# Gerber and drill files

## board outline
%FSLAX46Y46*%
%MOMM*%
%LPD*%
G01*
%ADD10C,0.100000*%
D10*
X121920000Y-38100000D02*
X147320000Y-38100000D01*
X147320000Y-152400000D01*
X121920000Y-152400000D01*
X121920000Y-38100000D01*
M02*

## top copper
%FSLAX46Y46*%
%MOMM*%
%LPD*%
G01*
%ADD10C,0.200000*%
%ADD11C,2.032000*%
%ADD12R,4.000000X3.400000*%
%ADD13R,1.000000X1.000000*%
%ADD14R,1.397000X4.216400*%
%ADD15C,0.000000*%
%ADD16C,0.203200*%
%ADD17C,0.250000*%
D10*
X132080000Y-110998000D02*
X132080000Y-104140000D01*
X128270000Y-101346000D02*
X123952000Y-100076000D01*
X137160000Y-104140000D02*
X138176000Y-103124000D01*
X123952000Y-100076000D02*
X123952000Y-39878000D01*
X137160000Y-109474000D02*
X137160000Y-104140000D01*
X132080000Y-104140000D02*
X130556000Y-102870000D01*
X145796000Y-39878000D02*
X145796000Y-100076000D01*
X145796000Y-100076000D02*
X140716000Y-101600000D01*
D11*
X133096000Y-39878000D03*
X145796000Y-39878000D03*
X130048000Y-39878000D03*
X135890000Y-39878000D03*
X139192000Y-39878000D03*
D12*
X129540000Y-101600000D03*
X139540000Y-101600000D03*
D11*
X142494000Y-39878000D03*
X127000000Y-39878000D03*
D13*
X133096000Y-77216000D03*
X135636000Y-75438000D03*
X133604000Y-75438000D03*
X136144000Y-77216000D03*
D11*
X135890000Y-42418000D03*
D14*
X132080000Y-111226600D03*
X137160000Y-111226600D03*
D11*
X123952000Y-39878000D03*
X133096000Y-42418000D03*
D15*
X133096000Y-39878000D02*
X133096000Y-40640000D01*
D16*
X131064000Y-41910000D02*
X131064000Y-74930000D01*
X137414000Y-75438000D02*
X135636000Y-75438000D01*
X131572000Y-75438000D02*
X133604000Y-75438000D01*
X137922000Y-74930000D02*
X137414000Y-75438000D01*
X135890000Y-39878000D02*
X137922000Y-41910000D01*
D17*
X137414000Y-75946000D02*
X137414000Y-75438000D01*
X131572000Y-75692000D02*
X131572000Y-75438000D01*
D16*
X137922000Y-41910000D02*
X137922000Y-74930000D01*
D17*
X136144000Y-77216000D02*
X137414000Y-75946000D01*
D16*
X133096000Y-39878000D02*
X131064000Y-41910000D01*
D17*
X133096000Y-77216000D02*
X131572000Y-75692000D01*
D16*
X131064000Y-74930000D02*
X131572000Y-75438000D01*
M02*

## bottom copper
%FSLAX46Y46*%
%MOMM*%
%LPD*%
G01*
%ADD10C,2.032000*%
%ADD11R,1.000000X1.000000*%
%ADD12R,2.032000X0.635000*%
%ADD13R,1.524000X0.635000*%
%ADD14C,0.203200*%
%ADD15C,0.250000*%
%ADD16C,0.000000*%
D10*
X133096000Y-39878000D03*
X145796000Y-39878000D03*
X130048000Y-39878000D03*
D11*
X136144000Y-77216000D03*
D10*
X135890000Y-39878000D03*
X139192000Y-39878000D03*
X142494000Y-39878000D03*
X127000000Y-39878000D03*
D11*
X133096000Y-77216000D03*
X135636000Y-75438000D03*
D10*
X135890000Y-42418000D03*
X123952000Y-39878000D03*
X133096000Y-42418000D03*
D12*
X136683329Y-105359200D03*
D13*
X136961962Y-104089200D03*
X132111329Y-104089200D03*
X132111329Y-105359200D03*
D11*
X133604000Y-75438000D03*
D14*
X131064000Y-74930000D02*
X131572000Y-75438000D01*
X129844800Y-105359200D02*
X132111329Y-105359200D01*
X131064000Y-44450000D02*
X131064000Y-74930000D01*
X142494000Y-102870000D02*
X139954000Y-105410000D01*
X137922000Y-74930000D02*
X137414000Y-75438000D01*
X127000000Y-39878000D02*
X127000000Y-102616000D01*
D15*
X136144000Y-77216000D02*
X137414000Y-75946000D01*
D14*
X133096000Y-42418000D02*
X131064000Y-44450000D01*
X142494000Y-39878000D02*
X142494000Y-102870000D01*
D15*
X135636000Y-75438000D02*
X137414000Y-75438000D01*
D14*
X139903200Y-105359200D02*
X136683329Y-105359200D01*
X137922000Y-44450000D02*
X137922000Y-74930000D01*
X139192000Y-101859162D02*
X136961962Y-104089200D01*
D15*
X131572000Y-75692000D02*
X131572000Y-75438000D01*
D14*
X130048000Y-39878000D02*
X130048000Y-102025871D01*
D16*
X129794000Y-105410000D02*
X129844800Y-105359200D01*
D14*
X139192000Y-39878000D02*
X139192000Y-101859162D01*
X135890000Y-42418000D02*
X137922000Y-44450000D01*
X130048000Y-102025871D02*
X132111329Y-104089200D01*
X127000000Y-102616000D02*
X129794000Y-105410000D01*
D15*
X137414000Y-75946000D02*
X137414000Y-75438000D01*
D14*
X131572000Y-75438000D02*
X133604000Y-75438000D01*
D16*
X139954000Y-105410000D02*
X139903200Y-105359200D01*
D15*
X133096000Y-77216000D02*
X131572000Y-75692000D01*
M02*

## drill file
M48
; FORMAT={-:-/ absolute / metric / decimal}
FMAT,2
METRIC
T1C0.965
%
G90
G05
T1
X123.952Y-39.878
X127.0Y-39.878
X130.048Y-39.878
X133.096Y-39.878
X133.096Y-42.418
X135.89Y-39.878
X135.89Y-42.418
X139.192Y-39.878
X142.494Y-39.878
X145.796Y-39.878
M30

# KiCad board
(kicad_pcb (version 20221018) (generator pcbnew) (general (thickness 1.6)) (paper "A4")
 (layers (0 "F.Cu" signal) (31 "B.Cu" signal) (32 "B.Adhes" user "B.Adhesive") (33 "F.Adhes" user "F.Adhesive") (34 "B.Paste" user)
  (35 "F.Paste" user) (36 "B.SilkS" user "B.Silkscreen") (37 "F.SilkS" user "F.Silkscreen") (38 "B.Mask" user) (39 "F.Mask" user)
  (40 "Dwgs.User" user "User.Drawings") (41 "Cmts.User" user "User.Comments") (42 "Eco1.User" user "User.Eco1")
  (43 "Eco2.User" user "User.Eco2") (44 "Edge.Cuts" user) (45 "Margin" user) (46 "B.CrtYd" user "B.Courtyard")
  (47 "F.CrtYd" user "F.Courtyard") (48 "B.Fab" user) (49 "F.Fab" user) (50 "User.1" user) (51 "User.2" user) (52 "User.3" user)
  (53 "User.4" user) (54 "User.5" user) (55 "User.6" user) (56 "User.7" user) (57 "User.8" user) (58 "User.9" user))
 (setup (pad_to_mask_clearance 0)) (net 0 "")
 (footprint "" (layer "F.Cu") (at 133.096 52.578)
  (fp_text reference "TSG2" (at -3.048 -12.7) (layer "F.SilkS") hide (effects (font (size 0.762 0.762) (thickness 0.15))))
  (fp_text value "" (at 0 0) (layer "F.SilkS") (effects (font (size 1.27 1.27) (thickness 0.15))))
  (pad "1" thru_hole circle (at 0 -12.7) (size 2.032 2.032) (drill 0.9652) (layers "*.Cu" "*.Mask")))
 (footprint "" (layer "F.Cu") (at 145.796 39.878)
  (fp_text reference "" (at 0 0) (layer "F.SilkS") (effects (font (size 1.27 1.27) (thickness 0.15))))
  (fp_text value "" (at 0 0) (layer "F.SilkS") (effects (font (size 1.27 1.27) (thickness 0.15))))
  (pad "1" thru_hole circle (at 0 0) (size 2.032 2.032) (drill 0.9652) (layers "*.Cu" "*.Mask")))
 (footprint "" (layer "F.Cu") (at 130.048 39.878)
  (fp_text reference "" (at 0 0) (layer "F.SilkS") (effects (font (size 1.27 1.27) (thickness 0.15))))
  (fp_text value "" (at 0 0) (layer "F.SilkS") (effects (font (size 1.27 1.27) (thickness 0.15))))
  (pad "1" thru_hole circle (at 0 0) (size 2.032 2.032) (drill 0.9652) (layers "*.Cu" "*.Mask")))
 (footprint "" (layer "F.Cu") (at 136.144 77.216)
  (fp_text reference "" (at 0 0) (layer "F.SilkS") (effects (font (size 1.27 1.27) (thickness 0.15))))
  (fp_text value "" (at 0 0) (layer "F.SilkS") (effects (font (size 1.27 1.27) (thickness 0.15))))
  (pad "1" smd rect (at 0 0 180) (size 1 1) (layers "B.Cu" "B.Mask")))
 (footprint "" (layer "F.Cu") (at 135.89 52.578)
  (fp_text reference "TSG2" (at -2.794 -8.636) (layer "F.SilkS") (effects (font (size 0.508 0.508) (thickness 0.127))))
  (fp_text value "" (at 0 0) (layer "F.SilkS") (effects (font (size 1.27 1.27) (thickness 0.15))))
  (pad "1" thru_hole circle (at 0 -12.7) (size 2.032 2.032) (drill 0.9652) (layers "*.Cu" "*.Mask")))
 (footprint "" (layer "F.Cu") (at 139.192 39.878)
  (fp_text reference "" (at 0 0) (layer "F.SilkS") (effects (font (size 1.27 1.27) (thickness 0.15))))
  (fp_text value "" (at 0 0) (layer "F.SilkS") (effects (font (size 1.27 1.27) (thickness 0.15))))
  (pad "1" thru_hole circle (at 0 0) (size 2.032 2.032) (drill 0.9652) (layers "*.Cu" "*.Mask")))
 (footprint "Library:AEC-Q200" (layer "F.Cu") (at 134.62 107.95)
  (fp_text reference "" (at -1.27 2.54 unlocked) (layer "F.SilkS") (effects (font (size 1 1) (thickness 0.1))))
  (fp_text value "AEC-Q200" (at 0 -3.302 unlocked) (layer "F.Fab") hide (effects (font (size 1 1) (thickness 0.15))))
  (pad "1" smd rect (at -5.08 -6.35 180) (size 4 3.4) (layers "F.Cu" "F.Mask"))
  (pad "2" smd rect (at 4.92 -6.35 180) (size 4 3.4) (layers "F.Cu" "F.Mask")))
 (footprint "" (layer "F.Cu") (at 142.494 39.878)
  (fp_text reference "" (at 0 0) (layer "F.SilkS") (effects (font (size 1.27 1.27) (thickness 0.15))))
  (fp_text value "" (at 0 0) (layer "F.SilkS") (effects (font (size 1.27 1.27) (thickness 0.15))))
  (pad "1" thru_hole circle (at 0 0) (size 2.032 2.032) (drill 0.9652) (layers "*.Cu" "*.Mask")))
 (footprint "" (layer "F.Cu") (at 127 39.878)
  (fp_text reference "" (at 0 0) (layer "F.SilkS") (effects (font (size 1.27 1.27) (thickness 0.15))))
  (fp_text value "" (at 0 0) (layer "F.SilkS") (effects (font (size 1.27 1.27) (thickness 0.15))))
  (pad "1" thru_hole circle (at 0 0) (size 2.032 2.032) (drill 0.9652) (layers "*.Cu" "*.Mask")))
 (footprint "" (layer "F.Cu") (at 133.096 77.216)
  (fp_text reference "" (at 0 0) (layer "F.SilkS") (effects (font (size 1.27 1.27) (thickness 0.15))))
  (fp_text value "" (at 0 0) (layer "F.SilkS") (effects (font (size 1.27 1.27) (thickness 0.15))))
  (pad "1" smd rect (at 0 0) (size 1 1) (layers "F.Cu" "F.Mask")))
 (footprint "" (layer "F.Cu") (at 133.096 77.216)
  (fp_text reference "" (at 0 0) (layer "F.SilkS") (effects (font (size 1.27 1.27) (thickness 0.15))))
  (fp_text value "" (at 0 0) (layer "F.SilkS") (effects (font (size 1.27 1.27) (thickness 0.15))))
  (pad "1" smd rect (at 0 0 180) (size 1 1) (layers "B.Cu" "B.Mask")))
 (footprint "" (layer "F.Cu") (at 135.636 75.438)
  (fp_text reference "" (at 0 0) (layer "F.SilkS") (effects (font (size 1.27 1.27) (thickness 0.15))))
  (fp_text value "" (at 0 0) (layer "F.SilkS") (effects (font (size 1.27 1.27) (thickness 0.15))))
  (pad "1" smd rect (at 0 0) (size 1 1) (layers "F.Cu" "F.Mask")))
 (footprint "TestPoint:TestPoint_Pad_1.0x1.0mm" (layer "F.Cu") (at 133.604 75.438)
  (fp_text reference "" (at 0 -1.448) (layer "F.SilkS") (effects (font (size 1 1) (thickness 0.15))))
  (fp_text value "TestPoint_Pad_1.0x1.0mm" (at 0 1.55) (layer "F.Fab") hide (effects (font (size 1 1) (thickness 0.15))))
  (pad "1" smd rect (at 0 0) (size 1 1) (layers "F.Cu" "F.Mask")))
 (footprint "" (layer "F.Cu") (at 136.144 77.216)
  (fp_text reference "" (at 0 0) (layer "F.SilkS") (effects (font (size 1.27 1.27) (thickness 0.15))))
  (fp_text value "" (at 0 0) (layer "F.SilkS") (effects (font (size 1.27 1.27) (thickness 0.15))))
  (pad "1" smd rect (at 0 0) (size 1 1) (layers "F.Cu" "F.Mask")))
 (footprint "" (layer "F.Cu") (at 135.636 75.438)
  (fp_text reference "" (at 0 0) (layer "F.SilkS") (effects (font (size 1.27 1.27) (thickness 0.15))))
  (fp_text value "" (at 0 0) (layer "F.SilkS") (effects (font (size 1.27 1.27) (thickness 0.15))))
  (pad "1" smd rect (at 0 0 180) (size 1 1) (layers "B.Cu" "B.Mask")))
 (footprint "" (layer "F.Cu") (at 135.89 55.118)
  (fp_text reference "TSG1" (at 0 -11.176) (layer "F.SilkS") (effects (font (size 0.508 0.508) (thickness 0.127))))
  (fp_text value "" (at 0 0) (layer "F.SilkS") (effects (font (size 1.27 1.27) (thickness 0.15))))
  (pad "1" thru_hole circle (at 0 -12.7) (size 2.032 2.032) (drill 0.9652) (layers "*.Cu" "*.Mask")))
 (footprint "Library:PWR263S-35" (layer "F.Cu") (at 135.89 112.268)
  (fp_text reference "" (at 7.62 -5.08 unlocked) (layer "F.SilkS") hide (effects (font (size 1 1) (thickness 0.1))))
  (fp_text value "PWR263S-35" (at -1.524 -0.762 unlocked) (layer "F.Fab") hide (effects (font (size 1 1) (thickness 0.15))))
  (pad "1" smd rect (at -3.81 -1.0414) (size 1.397 4.2164) (layers "F.Cu" "F.Mask"))
  (pad "2" smd rect (at 1.27 -1.0414) (size 1.397 4.2164) (layers "F.Cu" "F.Mask")))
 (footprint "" (layer "F.Cu") (at 123.952 39.878)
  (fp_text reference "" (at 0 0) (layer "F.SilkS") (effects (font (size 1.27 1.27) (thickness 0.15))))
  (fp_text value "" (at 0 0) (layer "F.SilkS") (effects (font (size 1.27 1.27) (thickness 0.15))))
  (pad "1" thru_hole circle (at 0 0) (size 2.032 2.032) (drill 0.9652) (layers "*.Cu" "*.Mask")))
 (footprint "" (layer "F.Cu") (at 133.096 55.118)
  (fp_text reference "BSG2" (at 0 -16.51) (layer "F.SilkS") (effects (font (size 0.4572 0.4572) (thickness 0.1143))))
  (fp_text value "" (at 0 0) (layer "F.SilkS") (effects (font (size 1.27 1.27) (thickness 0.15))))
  (pad "1" thru_hole circle (at 0 -12.7) (size 2.032 2.032) (drill 0.9652) (layers "*.Cu" "*.Mask")))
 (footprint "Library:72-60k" (layer "B.Cu") (at 132.873329 109.1692 180)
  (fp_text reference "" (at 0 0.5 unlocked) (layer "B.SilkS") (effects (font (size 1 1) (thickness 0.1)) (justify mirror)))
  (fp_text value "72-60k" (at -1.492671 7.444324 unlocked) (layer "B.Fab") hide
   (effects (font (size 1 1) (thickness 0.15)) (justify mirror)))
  (pad "1" smd rect (at -3.81 3.81) (size 2.032 0.635) (layers "B.Cu" "B.Mask"))
  (pad "2" smd rect (at -4.088633 5.08) (size 1.524 0.635) (layers "B.Cu" "B.Mask"))
  (pad "3" smd rect (at 0.762 5.08) (size 1.524 0.635) (layers "B.Cu" "B.Mask"))
  (pad "4" smd rect (at 0.762 3.81) (size 1.524 0.635) (layers "B.Cu" "B.Mask")))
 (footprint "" (layer "B.Cu") (at 133.604 75.438 180)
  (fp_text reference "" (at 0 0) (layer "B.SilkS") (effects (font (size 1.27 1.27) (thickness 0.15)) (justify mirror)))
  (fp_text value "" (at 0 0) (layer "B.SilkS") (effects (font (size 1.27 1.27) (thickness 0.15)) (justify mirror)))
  (pad "1" smd rect (at 0 0 180) (size 1 1) (layers "B.Cu" "B.Mask")))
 (gr_line (start 132.08 110.998) (end 132.08 104.14) (stroke (width 0.2) (type default)) (layer "F.Cu"))
 (gr_line (start 128.27 101.346) (end 123.952 100.076) (stroke (width 0.2) (type default)) (layer "F.Cu"))
 (gr_line (start 137.16 104.14) (end 138.176 103.124) (stroke (width 0.2) (type default)) (layer "F.Cu"))
 (gr_line (start 123.952 100.076) (end 123.952 39.878) (stroke (width 0.2) (type default)) (layer "F.Cu"))
 (gr_line (start 137.16 109.474) (end 137.16 104.14) (stroke (width 0.2) (type default)) (layer "F.Cu"))
 (gr_line (start 132.08 104.14) (end 130.556 102.87) (stroke (width 0.2) (type default)) (layer "F.Cu"))
 (gr_line (start 145.796 39.878) (end 145.796 100.076) (stroke (width 0.2) (type default)) (layer "F.Cu"))
 (gr_line (start 145.796 100.076) (end 140.716 101.6) (stroke (width 0.2) (type default)) (layer "F.Cu"))
 (gr_rect (start 121.92 38.1) (end 147.32 152.4) (stroke (width 0.1) (type default)) (fill none) (layer "Edge.Cuts"))
 (segment (start 133.096 39.878) (end 133.096 40.64) (width 0) (layer "F.Cu") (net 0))
 (segment (start 131.064 41.91) (end 131.064 74.93) (width 0.2032) (layer "F.Cu") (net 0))
 (segment (start 137.414 75.438) (end 135.636 75.438) (width 0.2032) (layer "F.Cu") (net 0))
 (segment (start 131.572 75.438) (end 133.604 75.438) (width 0.2032) (layer "F.Cu") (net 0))
 (segment (start 137.922 74.93) (end 137.414 75.438) (width 0.2032) (layer "F.Cu") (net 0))
 (segment (start 135.89 39.878) (end 137.922 41.91) (width 0.2032) (layer "F.Cu") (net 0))
 (segment (start 137.414 75.946) (end 137.414 75.438) (width 0.25) (layer "F.Cu") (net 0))
 (segment (start 131.572 75.692) (end 131.572 75.438) (width 0.25) (layer "F.Cu") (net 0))
 (segment (start 137.922 41.91) (end 137.922 74.93) (width 0.2032) (layer "F.Cu") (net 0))
 (segment (start 136.144 77.216) (end 137.414 75.946) (width 0.25) (layer "F.Cu") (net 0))
 (segment (start 133.096 39.878) (end 131.064 41.91) (width 0.2032) (layer "F.Cu") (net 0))
 (segment (start 133.096 77.216) (end 131.572 75.692) (width 0.25) (layer "F.Cu") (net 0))
 (segment (start 131.064 74.93) (end 131.572 75.438) (width 0.2032) (layer "F.Cu") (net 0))
 (segment (start 131.064 74.93) (end 131.572 75.438) (width 0.2032) (layer "B.Cu") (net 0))
 (segment (start 129.8448 105.3592) (end 132.111329 105.3592) (width 0.2032) (layer "B.Cu") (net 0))
 (segment (start 131.064 44.45) (end 131.064 74.93) (width 0.2032) (layer "B.Cu") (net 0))
 (segment (start 142.494 102.87) (end 139.954 105.41) (width 0.2032) (layer "B.Cu") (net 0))
 (segment (start 137.922 74.93) (end 137.414 75.438) (width 0.2032) (layer "B.Cu") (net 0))
 (segment (start 127 39.878) (end 127 102.616) (width 0.2032) (layer "B.Cu") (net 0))
 (segment (start 136.144 77.216) (end 137.414 75.946) (width 0.25) (layer "B.Cu") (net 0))
 (segment (start 133.096 42.418) (end 131.064 44.45) (width 0.2032) (layer "B.Cu") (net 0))
 (segment (start 142.494 39.878) (end 142.494 102.87) (width 0.2032) (layer "B.Cu") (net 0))
 (segment (start 135.636 75.438) (end 137.414 75.438) (width 0.25) (layer "B.Cu") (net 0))
 (segment (start 139.9032 105.3592) (end 136.683329 105.3592) (width 0.2032) (layer "B.Cu") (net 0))
 (segment (start 137.922 44.45) (end 137.922 74.93) (width 0.2032) (layer "B.Cu") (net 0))
 (segment (start 139.192 101.859162) (end 136.961962 104.0892) (width 0.2032) (layer "B.Cu") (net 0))
 (segment (start 131.572 75.692) (end 131.572 75.438) (width 0.25) (layer "B.Cu") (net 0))
 (segment (start 130.048 39.878) (end 130.048 102.025871) (width 0.2032) (layer "B.Cu") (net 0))
 (segment (start 129.794 105.41) (end 129.8448 105.3592) (width 0) (layer "B.Cu") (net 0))
 (segment (start 139.192 39.878) (end 139.192 101.859162) (width 0.2032) (layer "B.Cu") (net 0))
 (segment (start 135.89 42.418) (end 137.922 44.45) (width 0.2032) (layer "B.Cu") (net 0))
 (segment (start 130.048 102.025871) (end 132.111329 104.0892) (width 0.2032) (layer "B.Cu") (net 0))
 (segment (start 127 102.616) (end 129.794 105.41) (width 0.2032) (layer "B.Cu") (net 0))
 (segment (start 137.414 75.946) (end 137.414 75.438) (width 0.25) (layer "B.Cu") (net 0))
 (segment (start 131.572 75.438) (end 133.604 75.438) (width 0.2032) (layer "B.Cu") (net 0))
 (segment (start 139.954 105.41) (end 139.9032 105.3592) (width 0) (layer "B.Cu") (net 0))
 (segment (start 133.096 77.216) (end 131.572 75.692) (width 0.25) (layer "B.Cu") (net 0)))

